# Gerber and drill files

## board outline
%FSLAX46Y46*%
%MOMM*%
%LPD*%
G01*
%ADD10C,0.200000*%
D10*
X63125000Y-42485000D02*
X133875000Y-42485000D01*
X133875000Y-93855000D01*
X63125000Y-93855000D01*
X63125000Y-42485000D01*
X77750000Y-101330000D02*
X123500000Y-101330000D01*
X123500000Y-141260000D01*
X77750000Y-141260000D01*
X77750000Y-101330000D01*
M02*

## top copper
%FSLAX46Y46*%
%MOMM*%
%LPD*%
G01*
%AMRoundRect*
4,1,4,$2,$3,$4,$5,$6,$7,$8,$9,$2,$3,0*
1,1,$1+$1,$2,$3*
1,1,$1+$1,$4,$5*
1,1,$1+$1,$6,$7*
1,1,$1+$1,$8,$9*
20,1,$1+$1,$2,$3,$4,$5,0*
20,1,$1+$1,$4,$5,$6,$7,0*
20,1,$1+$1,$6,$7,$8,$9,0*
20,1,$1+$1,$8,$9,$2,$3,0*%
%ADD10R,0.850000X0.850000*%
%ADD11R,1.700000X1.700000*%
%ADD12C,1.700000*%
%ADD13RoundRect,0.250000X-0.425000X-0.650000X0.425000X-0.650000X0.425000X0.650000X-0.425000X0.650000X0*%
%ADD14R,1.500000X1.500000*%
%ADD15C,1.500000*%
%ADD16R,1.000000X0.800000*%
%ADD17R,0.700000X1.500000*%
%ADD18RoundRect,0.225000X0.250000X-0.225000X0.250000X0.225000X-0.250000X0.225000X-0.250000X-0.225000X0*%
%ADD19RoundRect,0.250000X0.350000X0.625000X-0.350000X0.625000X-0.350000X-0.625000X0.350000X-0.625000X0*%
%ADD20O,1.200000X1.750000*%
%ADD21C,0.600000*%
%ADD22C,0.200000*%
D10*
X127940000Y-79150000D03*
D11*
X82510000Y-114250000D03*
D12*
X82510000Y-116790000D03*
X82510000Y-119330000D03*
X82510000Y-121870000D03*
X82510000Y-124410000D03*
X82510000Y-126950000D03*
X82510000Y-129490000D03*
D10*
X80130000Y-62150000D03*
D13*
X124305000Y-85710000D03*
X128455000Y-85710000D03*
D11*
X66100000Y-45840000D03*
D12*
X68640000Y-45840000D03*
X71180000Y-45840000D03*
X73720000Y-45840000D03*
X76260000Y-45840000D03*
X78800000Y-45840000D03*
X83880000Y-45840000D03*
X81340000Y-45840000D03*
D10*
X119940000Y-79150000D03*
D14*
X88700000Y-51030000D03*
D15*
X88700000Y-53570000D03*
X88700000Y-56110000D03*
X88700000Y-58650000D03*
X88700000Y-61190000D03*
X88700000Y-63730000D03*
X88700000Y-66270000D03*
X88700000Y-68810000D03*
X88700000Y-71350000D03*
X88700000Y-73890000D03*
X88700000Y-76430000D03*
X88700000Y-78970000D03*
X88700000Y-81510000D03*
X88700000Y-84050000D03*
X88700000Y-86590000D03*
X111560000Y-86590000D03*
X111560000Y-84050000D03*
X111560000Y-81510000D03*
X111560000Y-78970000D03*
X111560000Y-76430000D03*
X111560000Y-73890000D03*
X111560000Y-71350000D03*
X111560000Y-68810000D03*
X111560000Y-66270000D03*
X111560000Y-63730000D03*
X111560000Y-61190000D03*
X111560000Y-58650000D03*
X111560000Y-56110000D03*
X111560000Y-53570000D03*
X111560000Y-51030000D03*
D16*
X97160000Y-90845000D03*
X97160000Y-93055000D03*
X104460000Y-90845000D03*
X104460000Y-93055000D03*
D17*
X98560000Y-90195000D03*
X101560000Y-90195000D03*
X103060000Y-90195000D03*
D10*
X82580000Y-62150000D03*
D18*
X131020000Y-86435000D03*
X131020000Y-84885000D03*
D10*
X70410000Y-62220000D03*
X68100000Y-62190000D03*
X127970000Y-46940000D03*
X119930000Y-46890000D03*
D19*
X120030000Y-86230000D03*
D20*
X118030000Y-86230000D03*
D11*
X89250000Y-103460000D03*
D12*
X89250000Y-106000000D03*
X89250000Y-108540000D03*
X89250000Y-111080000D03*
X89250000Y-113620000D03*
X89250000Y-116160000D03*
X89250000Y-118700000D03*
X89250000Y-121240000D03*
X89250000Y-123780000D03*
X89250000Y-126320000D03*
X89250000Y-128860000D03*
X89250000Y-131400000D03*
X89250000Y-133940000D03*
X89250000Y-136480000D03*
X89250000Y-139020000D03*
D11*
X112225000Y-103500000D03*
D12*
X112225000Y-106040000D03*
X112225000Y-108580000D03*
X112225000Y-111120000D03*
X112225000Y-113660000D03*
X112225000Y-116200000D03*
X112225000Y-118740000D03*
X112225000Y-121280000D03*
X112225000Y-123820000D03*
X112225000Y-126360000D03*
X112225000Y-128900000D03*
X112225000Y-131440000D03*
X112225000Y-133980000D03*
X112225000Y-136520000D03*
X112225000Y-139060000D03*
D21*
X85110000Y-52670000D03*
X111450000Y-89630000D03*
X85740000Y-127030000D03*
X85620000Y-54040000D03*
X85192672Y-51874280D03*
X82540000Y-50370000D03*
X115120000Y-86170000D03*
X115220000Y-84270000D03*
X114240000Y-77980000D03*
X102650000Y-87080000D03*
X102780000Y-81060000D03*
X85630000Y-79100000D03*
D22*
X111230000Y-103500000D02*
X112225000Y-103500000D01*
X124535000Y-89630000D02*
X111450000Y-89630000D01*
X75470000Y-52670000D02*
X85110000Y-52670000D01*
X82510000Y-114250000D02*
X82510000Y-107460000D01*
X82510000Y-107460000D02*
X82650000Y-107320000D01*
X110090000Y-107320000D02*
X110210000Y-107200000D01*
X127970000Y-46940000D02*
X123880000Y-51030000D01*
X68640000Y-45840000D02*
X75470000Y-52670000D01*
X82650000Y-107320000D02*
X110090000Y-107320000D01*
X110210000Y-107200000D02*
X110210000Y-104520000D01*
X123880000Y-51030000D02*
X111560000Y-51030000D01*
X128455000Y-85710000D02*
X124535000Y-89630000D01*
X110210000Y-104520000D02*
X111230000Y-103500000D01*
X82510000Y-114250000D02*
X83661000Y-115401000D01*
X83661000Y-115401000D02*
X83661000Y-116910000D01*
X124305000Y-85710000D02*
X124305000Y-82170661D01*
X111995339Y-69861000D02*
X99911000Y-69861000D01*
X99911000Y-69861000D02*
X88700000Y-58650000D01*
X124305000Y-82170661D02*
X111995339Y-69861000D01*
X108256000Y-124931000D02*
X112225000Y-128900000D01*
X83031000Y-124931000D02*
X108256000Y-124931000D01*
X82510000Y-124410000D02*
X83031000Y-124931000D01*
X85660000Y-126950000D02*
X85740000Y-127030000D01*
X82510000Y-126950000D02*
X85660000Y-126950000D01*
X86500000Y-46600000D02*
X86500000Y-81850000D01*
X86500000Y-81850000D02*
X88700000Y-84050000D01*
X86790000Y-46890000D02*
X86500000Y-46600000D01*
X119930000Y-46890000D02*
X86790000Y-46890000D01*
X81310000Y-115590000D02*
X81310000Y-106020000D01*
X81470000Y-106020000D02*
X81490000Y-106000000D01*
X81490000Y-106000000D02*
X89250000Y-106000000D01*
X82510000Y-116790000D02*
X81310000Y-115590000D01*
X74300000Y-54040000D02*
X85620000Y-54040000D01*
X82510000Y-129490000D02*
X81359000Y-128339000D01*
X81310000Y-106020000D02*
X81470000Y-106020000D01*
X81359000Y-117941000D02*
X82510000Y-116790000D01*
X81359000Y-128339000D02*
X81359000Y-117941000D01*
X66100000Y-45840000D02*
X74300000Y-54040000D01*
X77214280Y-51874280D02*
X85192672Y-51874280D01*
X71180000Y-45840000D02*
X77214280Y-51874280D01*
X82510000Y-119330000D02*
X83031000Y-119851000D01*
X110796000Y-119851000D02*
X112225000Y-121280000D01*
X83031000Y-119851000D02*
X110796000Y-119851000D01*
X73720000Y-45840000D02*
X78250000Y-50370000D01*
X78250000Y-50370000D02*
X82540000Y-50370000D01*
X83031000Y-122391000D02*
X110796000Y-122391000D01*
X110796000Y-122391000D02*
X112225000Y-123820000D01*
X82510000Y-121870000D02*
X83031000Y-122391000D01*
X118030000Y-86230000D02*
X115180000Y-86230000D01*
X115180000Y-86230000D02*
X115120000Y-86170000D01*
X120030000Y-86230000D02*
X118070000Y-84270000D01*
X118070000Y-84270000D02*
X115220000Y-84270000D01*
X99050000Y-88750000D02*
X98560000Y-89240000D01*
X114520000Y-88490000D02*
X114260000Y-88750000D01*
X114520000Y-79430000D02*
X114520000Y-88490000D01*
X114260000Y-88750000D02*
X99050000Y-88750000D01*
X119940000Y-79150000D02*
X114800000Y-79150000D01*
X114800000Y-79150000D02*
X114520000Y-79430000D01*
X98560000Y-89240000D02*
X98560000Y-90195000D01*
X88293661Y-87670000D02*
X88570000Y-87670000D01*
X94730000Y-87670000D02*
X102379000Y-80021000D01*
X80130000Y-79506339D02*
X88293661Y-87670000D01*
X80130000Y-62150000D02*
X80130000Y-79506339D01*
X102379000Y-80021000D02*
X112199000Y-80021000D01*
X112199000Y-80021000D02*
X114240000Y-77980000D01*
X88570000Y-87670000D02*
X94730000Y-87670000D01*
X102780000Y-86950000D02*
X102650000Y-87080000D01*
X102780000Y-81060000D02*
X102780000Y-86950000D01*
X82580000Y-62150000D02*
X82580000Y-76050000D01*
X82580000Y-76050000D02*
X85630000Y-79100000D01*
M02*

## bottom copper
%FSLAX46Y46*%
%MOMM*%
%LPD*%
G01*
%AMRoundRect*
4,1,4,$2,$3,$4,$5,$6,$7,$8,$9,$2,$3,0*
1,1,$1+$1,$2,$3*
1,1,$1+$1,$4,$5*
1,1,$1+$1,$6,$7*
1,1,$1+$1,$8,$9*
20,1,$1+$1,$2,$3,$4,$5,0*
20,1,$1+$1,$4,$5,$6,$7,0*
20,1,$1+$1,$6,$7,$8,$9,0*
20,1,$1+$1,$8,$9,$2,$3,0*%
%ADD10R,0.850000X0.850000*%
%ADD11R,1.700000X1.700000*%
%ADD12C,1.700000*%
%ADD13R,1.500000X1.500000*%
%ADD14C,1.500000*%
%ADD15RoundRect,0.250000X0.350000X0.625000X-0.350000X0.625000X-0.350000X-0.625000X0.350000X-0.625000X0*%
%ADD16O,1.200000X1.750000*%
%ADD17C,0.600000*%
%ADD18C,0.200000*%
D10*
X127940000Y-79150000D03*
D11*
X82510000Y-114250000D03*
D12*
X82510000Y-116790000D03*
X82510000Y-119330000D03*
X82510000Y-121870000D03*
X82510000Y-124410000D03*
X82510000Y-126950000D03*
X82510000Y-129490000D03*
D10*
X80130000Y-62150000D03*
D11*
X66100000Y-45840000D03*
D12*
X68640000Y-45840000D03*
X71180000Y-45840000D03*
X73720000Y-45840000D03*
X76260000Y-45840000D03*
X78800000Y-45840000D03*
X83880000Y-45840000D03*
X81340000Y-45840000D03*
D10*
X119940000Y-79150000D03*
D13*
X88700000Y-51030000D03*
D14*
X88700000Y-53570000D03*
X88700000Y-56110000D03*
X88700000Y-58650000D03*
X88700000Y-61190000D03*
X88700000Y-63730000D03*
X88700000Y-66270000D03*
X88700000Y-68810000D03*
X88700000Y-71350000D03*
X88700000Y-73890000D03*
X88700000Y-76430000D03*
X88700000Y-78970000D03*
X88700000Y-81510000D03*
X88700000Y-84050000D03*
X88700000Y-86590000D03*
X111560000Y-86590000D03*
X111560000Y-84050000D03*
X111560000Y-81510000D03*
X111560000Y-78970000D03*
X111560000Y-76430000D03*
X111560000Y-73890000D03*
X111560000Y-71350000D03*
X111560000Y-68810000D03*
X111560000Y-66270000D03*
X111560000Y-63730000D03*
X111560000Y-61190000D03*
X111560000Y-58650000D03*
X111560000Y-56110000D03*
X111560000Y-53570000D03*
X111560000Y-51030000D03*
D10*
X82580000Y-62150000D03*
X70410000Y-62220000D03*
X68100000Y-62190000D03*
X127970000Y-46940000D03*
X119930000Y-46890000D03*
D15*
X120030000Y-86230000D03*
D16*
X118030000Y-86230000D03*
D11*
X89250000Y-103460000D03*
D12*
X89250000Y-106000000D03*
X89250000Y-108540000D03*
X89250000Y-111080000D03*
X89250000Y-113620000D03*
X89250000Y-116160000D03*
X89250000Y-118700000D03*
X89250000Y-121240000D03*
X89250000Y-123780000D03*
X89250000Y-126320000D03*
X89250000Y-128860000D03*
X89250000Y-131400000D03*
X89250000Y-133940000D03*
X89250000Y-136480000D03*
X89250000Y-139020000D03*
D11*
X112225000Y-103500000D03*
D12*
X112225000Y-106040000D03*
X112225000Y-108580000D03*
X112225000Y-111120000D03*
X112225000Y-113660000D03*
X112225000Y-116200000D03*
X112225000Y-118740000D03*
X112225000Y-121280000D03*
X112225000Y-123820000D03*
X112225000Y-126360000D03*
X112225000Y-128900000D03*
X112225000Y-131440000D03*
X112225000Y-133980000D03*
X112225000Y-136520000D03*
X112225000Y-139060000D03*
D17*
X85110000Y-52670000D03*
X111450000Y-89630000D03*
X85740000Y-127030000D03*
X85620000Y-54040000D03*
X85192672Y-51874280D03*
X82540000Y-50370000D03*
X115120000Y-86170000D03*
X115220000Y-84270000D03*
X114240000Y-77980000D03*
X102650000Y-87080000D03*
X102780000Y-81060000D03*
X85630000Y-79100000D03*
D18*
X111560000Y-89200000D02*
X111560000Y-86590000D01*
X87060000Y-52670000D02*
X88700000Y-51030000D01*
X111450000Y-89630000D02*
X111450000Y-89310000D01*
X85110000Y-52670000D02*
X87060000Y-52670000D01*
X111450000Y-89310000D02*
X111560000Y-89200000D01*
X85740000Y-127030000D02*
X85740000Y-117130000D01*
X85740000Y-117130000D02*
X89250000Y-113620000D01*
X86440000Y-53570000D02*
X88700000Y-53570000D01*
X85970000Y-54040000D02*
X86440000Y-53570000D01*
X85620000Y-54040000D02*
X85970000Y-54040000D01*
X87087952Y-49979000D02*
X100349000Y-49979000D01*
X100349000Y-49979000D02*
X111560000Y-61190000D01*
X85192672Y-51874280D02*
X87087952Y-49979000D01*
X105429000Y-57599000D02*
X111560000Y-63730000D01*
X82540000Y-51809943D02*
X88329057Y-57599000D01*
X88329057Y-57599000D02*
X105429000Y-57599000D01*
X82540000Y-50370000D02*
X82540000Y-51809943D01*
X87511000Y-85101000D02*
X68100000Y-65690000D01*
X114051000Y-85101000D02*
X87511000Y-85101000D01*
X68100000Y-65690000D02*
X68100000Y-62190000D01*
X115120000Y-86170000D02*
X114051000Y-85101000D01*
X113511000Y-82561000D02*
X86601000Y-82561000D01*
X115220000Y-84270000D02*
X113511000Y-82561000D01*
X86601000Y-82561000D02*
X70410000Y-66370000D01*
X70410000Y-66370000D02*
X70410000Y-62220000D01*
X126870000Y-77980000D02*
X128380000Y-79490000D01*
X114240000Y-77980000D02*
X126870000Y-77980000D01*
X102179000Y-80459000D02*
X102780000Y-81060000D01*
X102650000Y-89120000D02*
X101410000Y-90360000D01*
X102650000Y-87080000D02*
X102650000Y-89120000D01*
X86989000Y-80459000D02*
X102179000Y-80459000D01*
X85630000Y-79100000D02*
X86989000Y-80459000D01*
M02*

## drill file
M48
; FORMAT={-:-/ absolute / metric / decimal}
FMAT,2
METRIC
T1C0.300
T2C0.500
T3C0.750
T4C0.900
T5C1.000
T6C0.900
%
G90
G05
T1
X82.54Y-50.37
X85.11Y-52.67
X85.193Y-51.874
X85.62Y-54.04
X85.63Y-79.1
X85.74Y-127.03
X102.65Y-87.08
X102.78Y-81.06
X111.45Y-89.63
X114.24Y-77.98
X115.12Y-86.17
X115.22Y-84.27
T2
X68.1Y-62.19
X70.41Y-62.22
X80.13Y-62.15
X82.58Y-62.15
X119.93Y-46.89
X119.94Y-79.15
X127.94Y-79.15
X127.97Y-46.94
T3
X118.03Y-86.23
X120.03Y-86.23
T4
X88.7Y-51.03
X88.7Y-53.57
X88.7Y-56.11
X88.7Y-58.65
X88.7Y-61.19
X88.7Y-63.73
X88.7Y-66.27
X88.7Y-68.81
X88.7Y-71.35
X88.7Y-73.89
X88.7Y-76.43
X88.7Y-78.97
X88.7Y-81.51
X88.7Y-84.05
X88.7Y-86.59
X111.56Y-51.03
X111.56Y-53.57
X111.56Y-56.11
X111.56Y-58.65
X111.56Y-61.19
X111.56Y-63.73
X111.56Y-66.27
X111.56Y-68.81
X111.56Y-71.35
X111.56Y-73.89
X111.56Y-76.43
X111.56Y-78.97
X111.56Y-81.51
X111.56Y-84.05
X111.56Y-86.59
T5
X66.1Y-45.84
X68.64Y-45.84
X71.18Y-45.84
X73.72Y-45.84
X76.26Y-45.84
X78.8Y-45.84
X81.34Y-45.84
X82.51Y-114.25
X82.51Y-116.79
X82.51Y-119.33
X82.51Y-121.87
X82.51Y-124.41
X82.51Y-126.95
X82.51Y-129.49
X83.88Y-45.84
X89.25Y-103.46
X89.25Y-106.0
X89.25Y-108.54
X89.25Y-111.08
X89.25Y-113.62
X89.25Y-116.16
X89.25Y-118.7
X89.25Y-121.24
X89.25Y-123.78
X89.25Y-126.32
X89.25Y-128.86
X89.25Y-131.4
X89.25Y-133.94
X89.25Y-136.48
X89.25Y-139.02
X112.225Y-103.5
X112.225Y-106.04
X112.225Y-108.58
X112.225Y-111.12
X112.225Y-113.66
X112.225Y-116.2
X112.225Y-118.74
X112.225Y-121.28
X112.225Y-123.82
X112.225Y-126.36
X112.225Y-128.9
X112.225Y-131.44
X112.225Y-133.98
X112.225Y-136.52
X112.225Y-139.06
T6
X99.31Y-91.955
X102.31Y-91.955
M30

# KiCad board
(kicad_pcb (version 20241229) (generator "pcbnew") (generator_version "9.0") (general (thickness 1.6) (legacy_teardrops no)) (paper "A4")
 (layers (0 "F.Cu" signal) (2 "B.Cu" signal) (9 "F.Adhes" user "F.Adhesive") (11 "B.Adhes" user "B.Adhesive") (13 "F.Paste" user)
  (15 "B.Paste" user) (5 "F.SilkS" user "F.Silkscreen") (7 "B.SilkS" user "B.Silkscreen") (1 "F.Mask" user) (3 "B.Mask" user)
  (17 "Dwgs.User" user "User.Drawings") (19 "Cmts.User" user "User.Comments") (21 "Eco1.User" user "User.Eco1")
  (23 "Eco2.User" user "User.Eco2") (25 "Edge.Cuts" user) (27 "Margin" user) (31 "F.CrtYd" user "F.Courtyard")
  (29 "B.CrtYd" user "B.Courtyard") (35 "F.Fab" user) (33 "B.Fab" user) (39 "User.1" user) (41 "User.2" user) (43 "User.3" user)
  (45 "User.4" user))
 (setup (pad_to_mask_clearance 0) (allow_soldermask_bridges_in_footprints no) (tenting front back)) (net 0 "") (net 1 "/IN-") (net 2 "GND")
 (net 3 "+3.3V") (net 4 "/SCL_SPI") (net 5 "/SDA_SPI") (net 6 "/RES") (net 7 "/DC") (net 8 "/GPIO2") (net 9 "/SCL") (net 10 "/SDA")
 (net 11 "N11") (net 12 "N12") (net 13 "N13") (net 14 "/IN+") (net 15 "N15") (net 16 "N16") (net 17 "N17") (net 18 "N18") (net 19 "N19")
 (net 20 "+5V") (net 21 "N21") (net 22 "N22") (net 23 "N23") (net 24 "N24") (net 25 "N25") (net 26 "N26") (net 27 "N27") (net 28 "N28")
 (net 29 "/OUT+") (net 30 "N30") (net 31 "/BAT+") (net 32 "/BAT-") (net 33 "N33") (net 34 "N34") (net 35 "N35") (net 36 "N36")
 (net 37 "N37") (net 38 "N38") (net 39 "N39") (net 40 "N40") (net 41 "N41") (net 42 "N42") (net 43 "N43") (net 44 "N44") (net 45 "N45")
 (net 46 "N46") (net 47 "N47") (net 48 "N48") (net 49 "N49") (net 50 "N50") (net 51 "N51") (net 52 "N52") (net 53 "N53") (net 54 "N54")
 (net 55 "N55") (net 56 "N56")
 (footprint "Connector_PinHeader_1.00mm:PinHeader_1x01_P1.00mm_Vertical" (layer "F.Cu") (at 127.94 79.15 90)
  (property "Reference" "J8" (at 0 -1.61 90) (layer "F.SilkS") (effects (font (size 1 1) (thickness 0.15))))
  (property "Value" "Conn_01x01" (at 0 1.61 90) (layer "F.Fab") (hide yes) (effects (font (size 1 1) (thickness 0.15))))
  (pad "1" thru_hole rect (at 0 0 90) (size 0.85 0.85) (drill 0.5) (layers "*.Cu" "*.Mask") (remove_unused_layers no) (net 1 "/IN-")))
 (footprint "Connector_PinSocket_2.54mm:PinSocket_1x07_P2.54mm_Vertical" (layer "F.Cu") (at 82.51 114.25)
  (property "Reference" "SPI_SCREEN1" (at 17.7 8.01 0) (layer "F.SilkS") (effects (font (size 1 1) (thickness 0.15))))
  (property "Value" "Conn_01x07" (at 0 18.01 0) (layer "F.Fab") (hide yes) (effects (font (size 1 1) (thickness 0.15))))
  (pad "1" thru_hole rect (at 0 0) (size 1.7 1.7) (drill 1) (layers "*.Cu" "*.Mask") (remove_unused_layers no) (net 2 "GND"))
  (pad "2" thru_hole circle (at 0 2.54) (size 1.7 1.7) (drill 1) (layers "*.Cu" "*.Mask") (remove_unused_layers no) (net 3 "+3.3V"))
  (pad "3" thru_hole circle (at 0 5.08) (size 1.7 1.7) (drill 1) (layers "*.Cu" "*.Mask") (remove_unused_layers no) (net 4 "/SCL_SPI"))
  (pad "4" thru_hole circle (at 0 7.62) (size 1.7 1.7) (drill 1) (layers "*.Cu" "*.Mask") (remove_unused_layers no) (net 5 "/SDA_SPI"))
  (pad "5" thru_hole circle (at 0 10.16) (size 1.7 1.7) (drill 1) (layers "*.Cu" "*.Mask") (remove_unused_layers no) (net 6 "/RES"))
  (pad "6" thru_hole circle (at 0 12.7) (size 1.7 1.7) (drill 1) (layers "*.Cu" "*.Mask") (remove_unused_layers no) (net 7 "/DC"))
  (pad "7" thru_hole circle (at 0 15.24) (size 1.7 1.7) (drill 1) (layers "*.Cu" "*.Mask") (remove_unused_layers no) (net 3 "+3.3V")))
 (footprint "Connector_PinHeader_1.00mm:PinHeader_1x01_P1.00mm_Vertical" (layer "F.Cu") (at 80.13 62.15 -90)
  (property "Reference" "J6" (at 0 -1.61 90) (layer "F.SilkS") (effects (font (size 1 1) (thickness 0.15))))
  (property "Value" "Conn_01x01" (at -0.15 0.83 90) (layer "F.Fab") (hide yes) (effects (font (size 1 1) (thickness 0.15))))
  (pad "1" thru_hole rect (at 0 0 270) (size 0.85 0.85) (drill 0.5) (layers "*.Cu" "*.Mask") (remove_unused_layers no) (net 1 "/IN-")))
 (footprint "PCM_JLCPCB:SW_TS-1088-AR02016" (layer "F.Cu") (at 126.38 85.71)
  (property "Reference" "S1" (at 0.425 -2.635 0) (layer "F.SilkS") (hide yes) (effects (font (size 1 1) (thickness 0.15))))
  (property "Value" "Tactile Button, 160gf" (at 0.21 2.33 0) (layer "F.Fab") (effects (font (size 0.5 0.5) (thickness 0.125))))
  (pad "1" smd roundrect (at -2.075 0) (size 1.35 1.8) (layers "F.Cu" "F.Mask" "F.Paste") (roundrect_rratio 0.1851851852) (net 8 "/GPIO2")
   (solder_mask_margin 0.102))
  (pad "2" smd roundrect (at 2.075 0) (size 1.35 1.8) (layers "F.Cu" "F.Mask" "F.Paste") (roundrect_rratio 0.1851851852) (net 2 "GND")
   (solder_mask_margin 0.102)))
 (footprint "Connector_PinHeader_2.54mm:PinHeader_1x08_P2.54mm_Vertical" (layer "F.Cu") (at 66.1 45.84 90)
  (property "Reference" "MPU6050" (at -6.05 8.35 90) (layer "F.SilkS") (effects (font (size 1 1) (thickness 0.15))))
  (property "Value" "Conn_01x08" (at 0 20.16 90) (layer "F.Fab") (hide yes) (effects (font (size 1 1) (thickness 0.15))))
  (pad "1" thru_hole rect (at 0 0 90) (size 1.7 1.7) (drill 1) (layers "*.Cu" "*.Mask") (remove_unused_layers no) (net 3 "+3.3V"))
  (pad "2" thru_hole circle (at 0 2.54 90) (size 1.7 1.7) (drill 1) (layers "*.Cu" "*.Mask") (remove_unused_layers no) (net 2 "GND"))
  (pad "3" thru_hole circle (at 0 5.08 90) (size 1.7 1.7) (drill 1) (layers "*.Cu" "*.Mask") (remove_unused_layers no) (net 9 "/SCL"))
  (pad "4" thru_hole circle (at 0 7.62 90) (size 1.7 1.7) (drill 1) (layers "*.Cu" "*.Mask") (remove_unused_layers no) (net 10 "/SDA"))
  (pad "5" thru_hole circle (at 0 10.16 90) (size 1.7 1.7) (drill 1) (layers "*.Cu" "*.Mask") (remove_unused_layers no) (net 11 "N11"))
  (pad "6" thru_hole circle (at 0 12.7 90) (size 1.7 1.7) (drill 1) (layers "*.Cu" "*.Mask") (remove_unused_layers no) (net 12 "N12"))
  (pad "8" thru_hole circle (at 0 17.78 90) (size 1.7 1.7) (drill 1) (layers "*.Cu" "*.Mask") (remove_unused_layers no) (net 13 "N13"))
  (pad "r" thru_hole circle (at 0 15.24 90) (size 1.7 1.7) (drill 1) (layers "*.Cu" "*.Mask") (remove_unused_layers no)))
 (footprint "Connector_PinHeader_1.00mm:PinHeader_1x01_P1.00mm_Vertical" (layer "F.Cu") (at 119.94 79.15 90)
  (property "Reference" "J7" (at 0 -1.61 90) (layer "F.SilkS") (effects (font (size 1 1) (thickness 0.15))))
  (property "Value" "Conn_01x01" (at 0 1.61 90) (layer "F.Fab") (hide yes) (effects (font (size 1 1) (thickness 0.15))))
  (pad "1" thru_hole rect (at 0 0 90) (size 0.85 0.85) (drill 0.5) (layers "*.Cu" "*.Mask") (remove_unused_layers no) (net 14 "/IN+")))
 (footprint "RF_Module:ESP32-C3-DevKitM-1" (layer "F.Cu") (at 88.7 51.03)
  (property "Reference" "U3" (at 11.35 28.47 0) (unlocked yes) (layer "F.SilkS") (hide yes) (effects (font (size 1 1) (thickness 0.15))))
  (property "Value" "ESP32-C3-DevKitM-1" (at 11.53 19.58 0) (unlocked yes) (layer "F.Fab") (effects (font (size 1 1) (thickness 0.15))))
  (pad "1" thru_hole rect (at 0 0) (size 1.5 1.5) (drill 0.9) (layers "*.Cu" "*.Mask") (remove_unused_layers yes) (keep_end_layers yes)
   (zone_layer_connections) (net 2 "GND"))
  (pad "2" thru_hole circle (at 0 2.54) (size 1.5 1.5) (drill 0.9) (layers "*.Cu" "*.Mask") (remove_unused_layers yes) (keep_end_layers yes)
   (zone_layer_connections) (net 3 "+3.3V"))
  (pad "3" thru_hole circle (at 0 5.08) (size 1.5 1.5) (drill 0.9) (layers "*.Cu" "*.Mask") (remove_unused_layers yes) (keep_end_layers yes)
   (zone_layer_connections) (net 3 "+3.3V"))
  (pad "4" thru_hole circle (at 0 7.62) (size 1.5 1.5) (drill 0.9) (layers "*.Cu" "*.Mask") (remove_unused_layers yes) (keep_end_layers yes)
   (zone_layer_connections) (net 8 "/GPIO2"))
  (pad "5" thru_hole circle (at 0 10.16) (size 1.5 1.5) (drill 0.9) (layers "*.Cu" "*.Mask") (remove_unused_layers yes)
   (keep_end_layers yes) (zone_layer_connections) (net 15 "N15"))
  (pad "6" thru_hole circle (at 0 12.7) (size 1.5 1.5) (drill 0.9) (layers "*.Cu" "*.Mask") (remove_unused_layers yes) (keep_end_layers yes)
   (zone_layer_connections) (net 2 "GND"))
  (pad "7" thru_hole circle (at 0 15.24) (size 1.5 1.5) (drill 0.9) (layers "*.Cu" "*.Mask") (remove_unused_layers yes)
   (keep_end_layers yes) (zone_layer_connections) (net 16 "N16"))
  (pad "8" thru_hole circle (at 0 17.78) (size 1.5 1.5) (drill 0.9) (layers "*.Cu" "*.Mask") (remove_unused_layers yes)
   (keep_end_layers yes) (zone_layer_connections) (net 2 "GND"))
  (pad "9" thru_hole circle (at 0 20.32) (size 1.5 1.5) (drill 0.9) (layers "*.Cu" "*.Mask") (remove_unused_layers yes)
   (keep_end_layers yes) (zone_layer_connections) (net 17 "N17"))
  (pad "10" thru_hole circle (at 0 22.86) (size 1.5 1.5) (drill 0.9) (layers "*.Cu" "*.Mask") (remove_unused_layers yes)
   (keep_end_layers yes) (zone_layer_connections) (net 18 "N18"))
  (pad "11" thru_hole circle (at 0 25.4) (size 1.5 1.5) (drill 0.9) (layers "*.Cu" "*.Mask") (remove_unused_layers yes)
   (keep_end_layers yes) (zone_layer_connections) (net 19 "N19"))
  (pad "12" thru_hole circle (at 0 27.94) (size 1.5 1.5) (drill 0.9) (layers "*.Cu" "*.Mask") (remove_unused_layers yes)
   (keep_end_layers yes) (zone_layer_connections) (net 2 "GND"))
  (pad "13" thru_hole circle (at 0 30.48) (size 1.5 1.5) (drill 0.9) (layers "*.Cu" "*.Mask") (remove_unused_layers yes)
   (keep_end_layers yes) (zone_layer_connections) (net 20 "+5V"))
  (pad "14" thru_hole circle (at 0 33.02) (size 1.5 1.5) (drill 0.9) (layers "*.Cu" "*.Mask") (remove_unused_layers yes)
   (keep_end_layers yes) (zone_layer_connections) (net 20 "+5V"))
  (pad "15" thru_hole circle (at 0 35.56) (size 1.5 1.5) (drill 0.9) (layers "*.Cu" "*.Mask") (remove_unused_layers yes)
   (keep_end_layers yes) (zone_layer_connections) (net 2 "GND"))
  (pad "16" thru_hole circle (at 22.86 35.56) (size 1.5 1.5) (drill 0.9) (layers "*.Cu" "*.Mask") (remove_unused_layers yes)
   (keep_end_layers yes) (zone_layer_connections) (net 2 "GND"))
  (pad "17" thru_hole circle (at 22.86 33.02) (size 1.5 1.5) (drill 0.9) (layers "*.Cu" "*.Mask") (remove_unused_layers yes)
   (keep_end_layers yes) (zone_layer_connections) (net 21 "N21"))
  (pad "18" thru_hole circle (at 22.86 30.48) (size 1.5 1.5) (drill 0.9) (layers "*.Cu" "*.Mask") (remove_unused_layers yes)
   (keep_end_layers yes) (zone_layer_connections) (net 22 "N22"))
  (pad "19" thru_hole circle (at 22.86 27.94) (size 1.5 1.5) (drill 0.9) (layers "*.Cu" "*.Mask") (remove_unused_layers yes)
   (keep_end_layers yes) (zone_layer_connections) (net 2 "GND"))
  (pad "20" thru_hole circle (at 22.86 25.4) (size 1.5 1.5) (drill 0.9) (layers "*.Cu" "*.Mask") (remove_unused_layers yes)
   (keep_end_layers yes) (zone_layer_connections) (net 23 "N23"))
  (pad "21" thru_hole circle (at 22.86 22.86) (size 1.5 1.5) (drill 0.9) (layers "*.Cu" "*.Mask") (remove_unused_layers yes)
   (keep_end_layers yes) (zone_layer_connections) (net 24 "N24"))
  (pad "22" thru_hole circle (at 22.86 20.32) (size 1.5 1.5) (drill 0.9) (layers "*.Cu" "*.Mask") (remove_unused_layers yes)
   (keep_end_layers yes) (zone_layer_connections) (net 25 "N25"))
  (pad "23" thru_hole circle (at 22.86 17.78) (size 1.5 1.5) (drill 0.9) (layers "*.Cu" "*.Mask") (remove_unused_layers yes)
   (keep_end_layers yes) (zone_layer_connections) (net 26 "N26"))
  (pad "24" thru_hole circle (at 22.86 15.24) (size 1.5 1.5) (drill 0.9) (layers "*.Cu" "*.Mask") (remove_unused_layers yes)
   (keep_end_layers yes) (zone_layer_connections) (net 2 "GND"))
  (pad "25" thru_hole circle (at 22.86 12.7) (size 1.5 1.5) (drill 0.9) (layers "*.Cu" "*.Mask") (remove_unused_layers yes)
   (keep_end_layers yes) (zone_layer_connections) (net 10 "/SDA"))
  (pad "26" thru_hole circle (at 22.86 10.16) (size 1.5 1.5) (drill 0.9) (layers "*.Cu" "*.Mask") (remove_unused_layers yes)
   (keep_end_layers yes) (zone_layer_connections) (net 9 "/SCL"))
  (pad "27" thru_hole circle (at 22.86 7.62) (size 1.5 1.5) (drill 0.9) (layers "*.Cu" "*.Mask") (remove_unused_layers yes)
   (keep_end_layers yes) (zone_layer_connections) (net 2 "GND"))
  (pad "28" thru_hole circle (at 22.86 5.08) (size 1.5 1.5) (drill 0.9) (layers "*.Cu" "*.Mask") (remove_unused_layers yes)
   (keep_end_layers yes) (zone_layer_connections) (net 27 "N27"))
  (pad "29" thru_hole circle (at 22.86 2.54) (size 1.5 1.5) (drill 0.9) (layers "*.Cu" "*.Mask") (remove_unused_layers yes)
   (keep_end_layers yes) (zone_layer_connections) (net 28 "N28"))
  (pad "30" thru_hole circle (at 22.86 0) (size 1.5 1.5) (drill 0.9) (layers "*.Cu" "*.Mask") (remove_unused_layers yes)
   (keep_end_layers yes) (zone_layer_connections) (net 2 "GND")))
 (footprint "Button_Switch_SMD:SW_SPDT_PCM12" (layer "F.Cu") (at 100.81 91.625)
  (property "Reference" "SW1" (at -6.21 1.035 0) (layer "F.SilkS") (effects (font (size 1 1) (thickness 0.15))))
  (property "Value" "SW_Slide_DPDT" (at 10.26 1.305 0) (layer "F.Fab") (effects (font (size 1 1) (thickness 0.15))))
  (pad "" smd rect (at -3.65 -0.78) (size 1 0.8) (layers "F.Cu" "F.Mask" "F.Paste"))
  (pad "" smd rect (at -3.65 1.43) (size 1 0.8) (layers "F.Cu" "F.Mask" "F.Paste"))
  (pad "" np_thru_hole circle (at -1.5 0.33) (size 0.9 0.9) (drill 0.9) (layers "*.Cu" "*.Mask"))
  (pad "" np_thru_hole circle (at 1.5 0.33) (size 0.9 0.9) (drill 0.9) (layers "*.Cu" "*.Mask"))
  (pad "" smd rect (at 3.65 -0.78) (size 1 0.8) (layers "F.Cu" "F.Mask" "F.Paste"))
  (pad "" smd rect (at 3.65 1.43) (size 1 0.8) (layers "F.Cu" "F.Mask" "F.Paste"))
  (pad "1" smd rect (at -2.25 -1.43) (size 0.7 1.5) (layers "F.Cu" "F.Mask" "F.Paste") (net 14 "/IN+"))
  (pad "2" smd rect (at 0.75 -1.43) (size 0.7 1.5) (layers "F.Cu" "F.Mask" "F.Paste") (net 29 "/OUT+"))
  (pad "3" smd rect (at 2.25 -1.43) (size 0.7 1.5) (layers "F.Cu" "F.Mask" "F.Paste") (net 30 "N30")))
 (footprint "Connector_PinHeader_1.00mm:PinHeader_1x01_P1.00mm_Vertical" (layer "F.Cu") (at 82.58 62.15 -90)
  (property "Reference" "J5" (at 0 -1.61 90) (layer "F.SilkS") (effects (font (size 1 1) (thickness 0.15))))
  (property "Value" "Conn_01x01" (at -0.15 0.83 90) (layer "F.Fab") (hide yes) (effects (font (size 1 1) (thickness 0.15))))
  (pad "1" thru_hole rect (at 0 0 270) (size 0.85 0.85) (drill 0.5) (layers "*.Cu" "*.Mask") (remove_unused_layers no) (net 29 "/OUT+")))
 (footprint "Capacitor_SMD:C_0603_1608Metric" (layer "F.Cu") (at 131.02 85.66 90)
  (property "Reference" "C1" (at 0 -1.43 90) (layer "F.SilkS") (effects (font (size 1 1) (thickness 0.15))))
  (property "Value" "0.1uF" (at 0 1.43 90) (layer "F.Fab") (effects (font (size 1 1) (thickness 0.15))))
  (pad "1" smd roundrect (at -0.775 0 90) (size 0.9 0.95) (layers "F.Cu" "F.Mask" "F.Paste") (roundrect_rratio 0.25) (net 3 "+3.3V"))
  (pad "2" smd roundrect (at 0.775 0 90) (size 0.9 0.95) (layers "F.Cu" "F.Mask" "F.Paste") (roundrect_rratio 0.25) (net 2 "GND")))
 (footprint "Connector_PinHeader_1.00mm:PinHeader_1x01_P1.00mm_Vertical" (layer "F.Cu") (at 70.41 62.22 -90)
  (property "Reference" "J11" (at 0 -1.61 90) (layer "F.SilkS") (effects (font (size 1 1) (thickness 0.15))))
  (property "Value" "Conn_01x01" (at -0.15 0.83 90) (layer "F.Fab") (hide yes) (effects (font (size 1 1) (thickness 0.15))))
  (pad "1" thru_hole rect (at 0 0 270) (size 0.85 0.85) (drill 0.5) (layers "*.Cu" "*.Mask") (remove_unused_layers no) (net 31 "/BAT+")))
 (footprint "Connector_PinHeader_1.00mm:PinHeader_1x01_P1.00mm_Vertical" (layer "F.Cu") (at 68.1 62.19 -90)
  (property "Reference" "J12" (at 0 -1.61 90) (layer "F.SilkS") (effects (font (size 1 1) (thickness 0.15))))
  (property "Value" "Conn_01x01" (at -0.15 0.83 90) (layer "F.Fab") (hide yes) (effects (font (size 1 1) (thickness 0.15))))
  (pad "1" thru_hole rect (at 0 0 270) (size 0.85 0.85) (drill 0.5) (layers "*.Cu" "*.Mask") (remove_unused_layers no) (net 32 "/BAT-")))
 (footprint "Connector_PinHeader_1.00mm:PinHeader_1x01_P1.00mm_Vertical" (layer "F.Cu") (at 127.97 46.94 90)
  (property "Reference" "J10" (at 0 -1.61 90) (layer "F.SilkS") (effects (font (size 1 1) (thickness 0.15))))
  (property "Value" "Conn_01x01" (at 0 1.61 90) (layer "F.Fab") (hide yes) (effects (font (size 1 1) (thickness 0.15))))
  (pad "1" thru_hole rect (at 0 0 90) (size 0.85 0.85) (drill 0.5) (layers "*.Cu" "*.Mask") (remove_unused_layers no) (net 2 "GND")))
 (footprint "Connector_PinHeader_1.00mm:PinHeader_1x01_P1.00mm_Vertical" (layer "F.Cu") (at 119.93 46.89 90)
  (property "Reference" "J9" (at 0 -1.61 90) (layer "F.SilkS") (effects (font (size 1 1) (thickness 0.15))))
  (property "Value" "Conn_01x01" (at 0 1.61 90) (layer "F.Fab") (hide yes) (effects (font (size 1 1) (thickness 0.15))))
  (pad "1" thru_hole rect (at 0 0 90) (size 0.85 0.85) (drill 0.5) (layers "*.Cu" "*.Mask") (remove_unused_layers no) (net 20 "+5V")))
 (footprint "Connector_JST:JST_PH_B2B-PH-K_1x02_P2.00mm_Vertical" (layer "F.Cu") (at 120.03 86.23 180)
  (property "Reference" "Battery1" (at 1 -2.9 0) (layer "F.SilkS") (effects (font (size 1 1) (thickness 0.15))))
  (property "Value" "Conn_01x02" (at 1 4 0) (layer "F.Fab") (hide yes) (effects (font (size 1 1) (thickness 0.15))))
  (pad "1" thru_hole roundrect (at 0 0 180) (size 1.2 1.75) (drill 0.75) (layers "*.Cu" "*.Mask") (remove_unused_layers no)
   (roundrect_rratio 0.208333) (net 31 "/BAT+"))
  (pad "2" thru_hole oval (at 2 0 180) (size 1.2 1.75) (drill 0.75) (layers "*.Cu" "*.Mask") (remove_unused_layers no) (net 32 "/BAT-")))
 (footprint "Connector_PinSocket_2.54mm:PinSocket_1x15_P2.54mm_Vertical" (layer "B.Cu") (at 89.25 103.46 180)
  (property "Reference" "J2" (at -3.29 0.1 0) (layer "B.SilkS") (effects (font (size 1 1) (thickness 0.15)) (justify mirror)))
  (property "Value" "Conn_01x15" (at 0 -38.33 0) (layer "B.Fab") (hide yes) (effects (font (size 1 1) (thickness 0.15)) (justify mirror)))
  (pad "1" thru_hole rect (at 0 0 180) (size 1.7 1.7) (drill 1) (layers "*.Cu" "*.Mask") (remove_unused_layers no) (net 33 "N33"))
  (pad "2" thru_hole circle (at 0 -2.54 180) (size 1.7 1.7) (drill 1) (layers "*.Cu" "*.Mask") (remove_unused_layers no) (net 3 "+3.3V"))
  (pad "3" thru_hole circle (at 0 -5.08 180) (size 1.7 1.7) (drill 1) (layers "*.Cu" "*.Mask") (remove_unused_layers no) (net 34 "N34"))
  (pad "4" thru_hole circle (at 0 -7.62 180) (size 1.7 1.7) (drill 1) (layers "*.Cu" "*.Mask") (remove_unused_layers no) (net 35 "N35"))
  (pad "5" thru_hole circle (at 0 -10.16 180) (size 1.7 1.7) (drill 1) (layers "*.Cu" "*.Mask") (remove_unused_layers no) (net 7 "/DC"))
  (pad "6" thru_hole circle (at 0 -12.7 180) (size 1.7 1.7) (drill 1) (layers "*.Cu" "*.Mask") (remove_unused_layers no) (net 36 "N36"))
  (pad "7" thru_hole circle (at 0 -15.24 180) (size 1.7 1.7) (drill 1) (layers "*.Cu" "*.Mask") (remove_unused_layers no) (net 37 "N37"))
  (pad "8" thru_hole circle (at 0 -17.78 180) (size 1.7 1.7) (drill 1) (layers "*.Cu" "*.Mask") (remove_unused_layers no) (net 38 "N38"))
  (pad "9" thru_hole circle (at 0 -20.32 180) (size 1.7 1.7) (drill 1) (layers "*.Cu" "*.Mask") (remove_unused_layers no) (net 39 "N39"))
  (pad "10" thru_hole circle (at 0 -22.86 180) (size 1.7 1.7) (drill 1) (layers "*.Cu" "*.Mask") (remove_unused_layers no) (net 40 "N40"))
  (pad "11" thru_hole circle (at 0 -25.4 180) (size 1.7 1.7) (drill 1) (layers "*.Cu" "*.Mask") (remove_unused_layers no) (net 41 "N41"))
  (pad "12" thru_hole circle (at 0 -27.94 180) (size 1.7 1.7) (drill 1) (layers "*.Cu" "*.Mask") (remove_unused_layers no) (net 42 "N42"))
  (pad "13" thru_hole circle (at 0 -30.48 180) (size 1.7 1.7) (drill 1) (layers "*.Cu" "*.Mask") (remove_unused_layers no) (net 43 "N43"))
  (pad "14" thru_hole circle (at 0 -33.02 180) (size 1.7 1.7) (drill 1) (layers "*.Cu" "*.Mask") (remove_unused_layers no) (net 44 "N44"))
  (pad "15" thru_hole circle (at 0 -35.56 180) (size 1.7 1.7) (drill 1) (layers "*.Cu" "*.Mask") (remove_unused_layers no) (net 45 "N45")))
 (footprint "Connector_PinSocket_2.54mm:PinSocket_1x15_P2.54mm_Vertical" (layer "B.Cu") (at 112.225 103.5 180)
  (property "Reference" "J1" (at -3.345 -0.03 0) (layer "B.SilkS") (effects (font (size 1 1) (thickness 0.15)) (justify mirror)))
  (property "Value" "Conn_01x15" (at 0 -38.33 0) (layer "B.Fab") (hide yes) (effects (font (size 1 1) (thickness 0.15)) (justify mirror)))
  (pad "1" thru_hole rect (at 0 0 180) (size 1.7 1.7) (drill 1) (layers "*.Cu" "*.Mask") (remove_unused_layers no) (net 2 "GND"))
  (pad "2" thru_hole circle (at 0 -2.54 180) (size 1.7 1.7) (drill 1) (layers "*.Cu" "*.Mask") (remove_unused_layers no) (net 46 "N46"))
  (pad "3" thru_hole circle (at 0 -5.08 180) (size 1.7 1.7) (drill 1) (layers "*.Cu" "*.Mask") (remove_unused_layers no) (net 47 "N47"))
  (pad "4" thru_hole circle (at 0 -7.62 180) (size 1.7 1.7) (drill 1) (layers "*.Cu" "*.Mask") (remove_unused_layers no) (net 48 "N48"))
  (pad "5" thru_hole circle (at 0 -10.16 180) (size 1.7 1.7) (drill 1) (layers "*.Cu" "*.Mask") (remove_unused_layers no) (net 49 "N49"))
  (pad "6" thru_hole circle (at 0 -12.7 180) (size 1.7 1.7) (drill 1) (layers "*.Cu" "*.Mask") (remove_unused_layers no) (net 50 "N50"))
  (pad "7" thru_hole circle (at 0 -15.24 180) (size 1.7 1.7) (drill 1) (layers "*.Cu" "*.Mask") (remove_unused_layers no) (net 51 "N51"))
  (pad "8" thru_hole circle (at 0 -17.78 180) (size 1.7 1.7) (drill 1) (layers "*.Cu" "*.Mask") (remove_unused_layers no) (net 4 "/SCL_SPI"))
  (pad "9" thru_hole circle (at 0 -20.32 180) (size 1.7 1.7) (drill 1) (layers "*.Cu" "*.Mask") (remove_unused_layers no) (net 5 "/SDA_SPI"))
  (pad "10" thru_hole circle (at 0 -22.86 180) (size 1.7 1.7) (drill 1) (layers "*.Cu" "*.Mask") (remove_unused_layers no) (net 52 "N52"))
  (pad "11" thru_hole circle (at 0 -25.4 180) (size 1.7 1.7) (drill 1) (layers "*.Cu" "*.Mask") (remove_unused_layers no) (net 6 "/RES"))
  (pad "12" thru_hole circle (at 0 -27.94 180) (size 1.7 1.7) (drill 1) (layers "*.Cu" "*.Mask") (remove_unused_layers no) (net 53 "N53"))
  (pad "13" thru_hole circle (at 0 -30.48 180) (size 1.7 1.7) (drill 1) (layers "*.Cu" "*.Mask") (remove_unused_layers no) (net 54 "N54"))
  (pad "14" thru_hole circle (at 0 -33.02 180) (size 1.7 1.7) (drill 1) (layers "*.Cu" "*.Mask") (remove_unused_layers no) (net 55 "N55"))
  (pad "15" thru_hole circle (at 0 -35.56 180) (size 1.7 1.7) (drill 1) (layers "*.Cu" "*.Mask") (remove_unused_layers no) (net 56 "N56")))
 (gr_rect (start 63.125 42.485) (end 133.875 93.855) (stroke (width 0.2) (type solid)) (fill no) (layer "Edge.Cuts"))
 (gr_rect (start 77.75 101.33) (end 123.5 141.26) (stroke (width 0.2) (type solid)) (fill no) (layer "Edge.Cuts"))
 (segment (start 111.23 103.5) (end 112.225 103.5) (width 0.2) (layer "F.Cu") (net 2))
 (segment (start 124.535 89.63) (end 111.45 89.63) (width 0.2) (layer "F.Cu") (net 2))
 (segment (start 75.47 52.67) (end 85.11 52.67) (width 0.2) (layer "F.Cu") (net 2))
 (segment (start 82.51 114.25) (end 82.51 107.46) (width 0.2) (layer "F.Cu") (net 2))
 (segment (start 82.51 107.46) (end 82.65 107.32) (width 0.2) (layer "F.Cu") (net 2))
 (segment (start 110.09 107.32) (end 110.21 107.2) (width 0.2) (layer "F.Cu") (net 2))
 (segment (start 127.97 46.94) (end 123.88 51.03) (width 0.2) (layer "F.Cu") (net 2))
 (segment (start 68.64 45.84) (end 75.47 52.67) (width 0.2) (layer "F.Cu") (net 2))
 (segment (start 82.65 107.32) (end 110.09 107.32) (width 0.2) (layer "F.Cu") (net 2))
 (segment (start 110.21 107.2) (end 110.21 104.52) (width 0.2) (layer "F.Cu") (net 2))
 (segment (start 123.88 51.03) (end 111.56 51.03) (width 0.2) (layer "F.Cu") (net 2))
 (segment (start 128.455 85.71) (end 124.535 89.63) (width 0.2) (layer "F.Cu") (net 2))
 (segment (start 110.21 104.52) (end 111.23 103.5) (width 0.2) (layer "F.Cu") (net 2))
 (segment (start 82.51 114.25) (end 83.661 115.401) (width 0.2) (layer "F.Cu") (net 2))
 (segment (start 83.661 115.401) (end 83.661 116.91) (width 0.2) (layer "F.Cu") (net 2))
 (via (at 85.11 52.67) (size 0.6) (drill 0.3) (layers "F.Cu" "B.Cu") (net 2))
 (via (at 111.45 89.63) (size 0.6) (drill 0.3) (layers "F.Cu" "B.Cu") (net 2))
 (segment (start 111.56 89.2) (end 111.56 86.59) (width 0.2) (layer "B.Cu") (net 2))
 (segment (start 87.06 52.67) (end 88.7 51.03) (width 0.2) (layer "B.Cu") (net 2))
 (segment (start 111.45 89.63) (end 111.45 89.31) (width 0.2) (layer "B.Cu") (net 2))
 (segment (start 85.11 52.67) (end 87.06 52.67) (width 0.2) (layer "B.Cu") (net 2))
 (segment (start 111.45 89.31) (end 111.56 89.2) (width 0.2) (layer "B.Cu") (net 2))
 (segment (start 124.305 85.71) (end 124.305 82.170661) (width 0.2) (layer "F.Cu") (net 8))
 (segment (start 111.995339 69.861) (end 99.911 69.861) (width 0.2) (layer "F.Cu") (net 8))
 (segment (start 99.911 69.861) (end 88.7 58.65) (width 0.2) (layer "F.Cu") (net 8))
 (segment (start 124.305 82.170661) (end 111.995339 69.861) (width 0.2) (layer "F.Cu") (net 8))
 (segment (start 108.256 124.931) (end 112.225 128.9) (width 0.2) (layer "F.Cu") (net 6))
 (segment (start 83.031 124.931) (end 108.256 124.931) (width 0.2) (layer "F.Cu") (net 6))
 (segment (start 82.51 124.41) (end 83.031 124.931) (width 0.2) (layer "F.Cu") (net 6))
 (segment (start 85.66 126.95) (end 85.74 127.03) (width 0.2) (layer "F.Cu") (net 7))
 (segment (start 82.51 126.95) (end 85.66 126.95) (width 0.2) (layer "F.Cu") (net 7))
 (via (at 85.74 127.03) (size 0.6) (drill 0.3) (layers "F.Cu" "B.Cu") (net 7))
 (segment (start 85.74 127.03) (end 85.74 117.13) (width 0.2) (layer "B.Cu") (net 7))
 (segment (start 85.74 117.13) (end 89.25 113.62) (width 0.2) (layer "B.Cu") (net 7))
 (segment (start 86.5 46.6) (end 86.5 81.85) (width 0.2) (layer "F.Cu") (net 20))
 (segment (start 86.5 81.85) (end 88.7 84.05) (width 0.2) (layer "F.Cu") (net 20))
 (segment (start 86.79 46.89) (end 86.5 46.6) (width 0.2) (layer "F.Cu") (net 20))
 (segment (start 119.93 46.89) (end 86.79 46.89) (width 0.2) (layer "F.Cu") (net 20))
 (segment (start 81.31 115.59) (end 81.31 106.02) (width 0.2) (layer "F.Cu") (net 3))
 (segment (start 81.47 106.02) (end 81.49 106) (width 0.2) (layer "F.Cu") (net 3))
 (segment (start 81.49 106) (end 89.25 106) (width 0.2) (layer "F.Cu") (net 3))
 (segment (start 82.51 116.79) (end 81.31 115.59) (width 0.2) (layer "F.Cu") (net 3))
 (segment (start 74.3 54.04) (end 85.62 54.04) (width 0.2) (layer "F.Cu") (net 3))
 (segment (start 82.51 129.49) (end 81.359 128.339) (width 0.2) (layer "F.Cu") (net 3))
 (segment (start 81.31 106.02) (end 81.47 106.02) (width 0.2) (layer "F.Cu") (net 3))
 (segment (start 81.359 117.941) (end 82.51 116.79) (width 0.2) (layer "F.Cu") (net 3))
 (segment (start 81.359 128.339) (end 81.359 117.941) (width 0.2) (layer "F.Cu") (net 3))
 (segment (start 66.1 45.84) (end 74.3 54.04) (width 0.2) (layer "F.Cu") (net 3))
 (via (at 85.62 54.04) (size 0.6) (drill 0.3) (layers "F.Cu" "B.Cu") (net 3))
 (segment (start 86.44 53.57) (end 88.7 53.57) (width 0.2) (layer "B.Cu") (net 3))
 (segment (start 85.97 54.04) (end 86.44 53.57) (width 0.2) (layer "B.Cu") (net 3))
 (segment (start 85.62 54.04) (end 85.97 54.04) (width 0.2) (layer "B.Cu") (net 3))
 (segment (start 77.21428 51.87428) (end 85.192672 51.87428) (width 0.2) (layer "F.Cu") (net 9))
 (segment (start 71.18 45.84) (end 77.21428 51.87428) (width 0.2) (layer "F.Cu") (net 9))
 (via (at 85.192672 51.87428) (size 0.6) (drill 0.3) (layers "F.Cu" "B.Cu") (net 9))
 (segment (start 87.087952 49.979) (end 100.349 49.979) (width 0.2) (layer "B.Cu") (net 9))
 (segment (start 100.349 49.979) (end 111.56 61.19) (width 0.2) (layer "B.Cu") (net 9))
 (segment (start 85.192672 51.87428) (end 87.087952 49.979) (width 0.2) (layer "B.Cu") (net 9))
 (segment (start 82.51 119.33) (end 83.031 119.851) (width 0.2) (layer "F.Cu") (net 4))
 (segment (start 110.796 119.851) (end 112.225 121.28) (width 0.2) (layer "F.Cu") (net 4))
 (segment (start 83.031 119.851) (end 110.796 119.851) (width 0.2) (layer "F.Cu") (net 4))
 (segment (start 73.72 45.84) (end 78.25 50.37) (width 0.2) (layer "F.Cu") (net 10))
 (segment (start 78.25 50.37) (end 82.54 50.37) (width 0.2) (layer "F.Cu") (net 10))
 (via (at 82.54 50.37) (size 0.6) (drill 0.3) (layers "F.Cu" "B.Cu") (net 10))
 (segment (start 105.429 57.599) (end 111.56 63.73) (width 0.2) (layer "B.Cu") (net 10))
 (segment (start 82.54 51.809943) (end 88.329057 57.599) (width 0.2) (layer "B.Cu") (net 10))
 (segment (start 88.329057 57.599) (end 105.429 57.599) (width 0.2) (layer "B.Cu") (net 10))
 (segment (start 82.54 50.37) (end 82.54 51.809943) (width 0.2) (layer "B.Cu") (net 10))
 (segment (start 83.031 122.391) (end 110.796 122.391) (width 0.2) (layer "F.Cu") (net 5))
 (segment (start 110.796 122.391) (end 112.225 123.82) (width 0.2) (layer "F.Cu") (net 5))
 (segment (start 82.51 121.87) (end 83.031 122.391) (width 0.2) (layer "F.Cu") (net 5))
 (segment (start 118.03 86.23) (end 115.18 86.23) (width 0.2) (layer "F.Cu") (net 32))
 (segment (start 115.18 86.23) (end 115.12 86.17) (width 0.2) (layer "F.Cu") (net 32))
 (via (at 115.12 86.17) (size 0.6) (drill 0.3) (layers "F.Cu" "B.Cu") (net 32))
 (segment (start 87.511 85.101) (end 68.1 65.69) (width 0.2) (layer "B.Cu") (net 32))
 (segment (start 114.051 85.101) (end 87.511 85.101) (width 0.2) (layer "B.Cu") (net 32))
 (segment (start 68.1 65.69) (end 68.1 62.19) (width 0.2) (layer "B.Cu") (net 32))
 (segment (start 115.12 86.17) (end 114.051 85.101) (width 0.2) (layer "B.Cu") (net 32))
 (segment (start 120.03 86.23) (end 118.07 84.27) (width 0.2) (layer "F.Cu") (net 31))
 (segment (start 118.07 84.27) (end 115.22 84.27) (width 0.2) (layer "F.Cu") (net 31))
 (via (at 115.22 84.27) (size 0.6) (drill 0.3) (layers "F.Cu" "B.Cu") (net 31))
 (segment (start 113.511 82.561) (end 86.601 82.561) (width 0.2) (layer "B.Cu") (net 31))
 (segment (start 115.22 84.27) (end 113.511 82.561) (width 0.2) (layer "B.Cu") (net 31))
 (segment (start 86.601 82.561) (end 70.41 66.37) (width 0.2) (layer "B.Cu") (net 31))
 (segment (start 70.41 66.37) (end 70.41 62.22) (width 0.2) (layer "B.Cu") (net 31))
 (segment (start 99.05 88.75) (end 98.56 89.24) (width 0.2) (layer "F.Cu") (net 14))
 (segment (start 114.52 88.49) (end 114.26 88.75) (width 0.2) (layer "F.Cu") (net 14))
 (segment (start 114.52 79.43) (end 114.52 88.49) (width 0.2) (layer "F.Cu") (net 14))
 (segment (start 114.26 88.75) (end 99.05 88.75) (width 0.2) (layer "F.Cu") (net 14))
 (segment (start 119.94 79.15) (end 114.8 79.15) (width 0.2) (layer "F.Cu") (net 14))
 (segment (start 114.8 79.15) (end 114.52 79.43) (width 0.2) (layer "F.Cu") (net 14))
 (segment (start 98.56 89.24) (end 98.56 90.195) (width 0.2) (layer "F.Cu") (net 14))
 (segment (start 88.293661 87.67) (end 88.57 87.67) (width 0.2) (layer "F.Cu") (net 1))
 (segment (start 94.73 87.67) (end 102.379 80.021) (width 0.2) (layer "F.Cu") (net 1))
 (segment (start 80.13 79.506339) (end 88.293661 87.67) (width 0.2) (layer "F.Cu") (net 1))
 (segment (start 80.13 62.15) (end 80.13 79.506339) (width 0.2) (layer "F.Cu") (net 1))
 (segment (start 102.379 80.021) (end 112.199 80.021) (width 0.2) (layer "F.Cu") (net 1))
 (segment (start 112.199 80.021) (end 114.24 77.98) (width 0.2) (layer "F.Cu") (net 1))
 (segment (start 88.57 87.67) (end 94.73 87.67) (width 0.2) (layer "F.Cu") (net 1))
 (via (at 114.24 77.98) (size 0.6) (drill 0.3) (layers "F.Cu" "B.Cu") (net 1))
 (segment (start 126.87 77.98) (end 128.38 79.49) (width 0.2) (layer "B.Cu") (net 1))
 (segment (start 114.24 77.98) (end 126.87 77.98) (width 0.2) (layer "B.Cu") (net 1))
 (segment (start 102.78 86.95) (end 102.65 87.08) (width 0.2) (layer "F.Cu") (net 29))
 (segment (start 102.78 81.06) (end 102.78 86.95) (width 0.2) (layer "F.Cu") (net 29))
 (segment (start 82.58 62.15) (end 82.58 76.05) (width 0.2) (layer "F.Cu") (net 29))
 (segment (start 82.58 76.05) (end 85.63 79.1) (width 0.2) (layer "F.Cu") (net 29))
 (via (at 102.65 87.08) (size 0.6) (drill 0.3) (layers "F.Cu" "B.Cu") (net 29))
 (via (at 102.78 81.06) (size 0.6) (drill 0.3) (layers "F.Cu" "B.Cu") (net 29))
 (via (at 85.63 79.1) (size 0.6) (drill 0.3) (layers "F.Cu" "B.Cu") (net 29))
 (segment (start 102.179 80.459) (end 102.78 81.06) (width 0.2) (layer "B.Cu") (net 29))
 (segment (start 102.65 89.12) (end 101.41 90.36) (width 0.2) (layer "B.Cu") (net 29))
 (segment (start 102.65 87.08) (end 102.65 89.12) (width 0.2) (layer "B.Cu") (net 29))
 (segment (start 86.989 80.459) (end 102.179 80.459) (width 0.2) (layer "B.Cu") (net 29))
 (segment (start 85.63 79.1) (end 86.989 80.459) (width 0.2) (layer "B.Cu") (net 29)))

